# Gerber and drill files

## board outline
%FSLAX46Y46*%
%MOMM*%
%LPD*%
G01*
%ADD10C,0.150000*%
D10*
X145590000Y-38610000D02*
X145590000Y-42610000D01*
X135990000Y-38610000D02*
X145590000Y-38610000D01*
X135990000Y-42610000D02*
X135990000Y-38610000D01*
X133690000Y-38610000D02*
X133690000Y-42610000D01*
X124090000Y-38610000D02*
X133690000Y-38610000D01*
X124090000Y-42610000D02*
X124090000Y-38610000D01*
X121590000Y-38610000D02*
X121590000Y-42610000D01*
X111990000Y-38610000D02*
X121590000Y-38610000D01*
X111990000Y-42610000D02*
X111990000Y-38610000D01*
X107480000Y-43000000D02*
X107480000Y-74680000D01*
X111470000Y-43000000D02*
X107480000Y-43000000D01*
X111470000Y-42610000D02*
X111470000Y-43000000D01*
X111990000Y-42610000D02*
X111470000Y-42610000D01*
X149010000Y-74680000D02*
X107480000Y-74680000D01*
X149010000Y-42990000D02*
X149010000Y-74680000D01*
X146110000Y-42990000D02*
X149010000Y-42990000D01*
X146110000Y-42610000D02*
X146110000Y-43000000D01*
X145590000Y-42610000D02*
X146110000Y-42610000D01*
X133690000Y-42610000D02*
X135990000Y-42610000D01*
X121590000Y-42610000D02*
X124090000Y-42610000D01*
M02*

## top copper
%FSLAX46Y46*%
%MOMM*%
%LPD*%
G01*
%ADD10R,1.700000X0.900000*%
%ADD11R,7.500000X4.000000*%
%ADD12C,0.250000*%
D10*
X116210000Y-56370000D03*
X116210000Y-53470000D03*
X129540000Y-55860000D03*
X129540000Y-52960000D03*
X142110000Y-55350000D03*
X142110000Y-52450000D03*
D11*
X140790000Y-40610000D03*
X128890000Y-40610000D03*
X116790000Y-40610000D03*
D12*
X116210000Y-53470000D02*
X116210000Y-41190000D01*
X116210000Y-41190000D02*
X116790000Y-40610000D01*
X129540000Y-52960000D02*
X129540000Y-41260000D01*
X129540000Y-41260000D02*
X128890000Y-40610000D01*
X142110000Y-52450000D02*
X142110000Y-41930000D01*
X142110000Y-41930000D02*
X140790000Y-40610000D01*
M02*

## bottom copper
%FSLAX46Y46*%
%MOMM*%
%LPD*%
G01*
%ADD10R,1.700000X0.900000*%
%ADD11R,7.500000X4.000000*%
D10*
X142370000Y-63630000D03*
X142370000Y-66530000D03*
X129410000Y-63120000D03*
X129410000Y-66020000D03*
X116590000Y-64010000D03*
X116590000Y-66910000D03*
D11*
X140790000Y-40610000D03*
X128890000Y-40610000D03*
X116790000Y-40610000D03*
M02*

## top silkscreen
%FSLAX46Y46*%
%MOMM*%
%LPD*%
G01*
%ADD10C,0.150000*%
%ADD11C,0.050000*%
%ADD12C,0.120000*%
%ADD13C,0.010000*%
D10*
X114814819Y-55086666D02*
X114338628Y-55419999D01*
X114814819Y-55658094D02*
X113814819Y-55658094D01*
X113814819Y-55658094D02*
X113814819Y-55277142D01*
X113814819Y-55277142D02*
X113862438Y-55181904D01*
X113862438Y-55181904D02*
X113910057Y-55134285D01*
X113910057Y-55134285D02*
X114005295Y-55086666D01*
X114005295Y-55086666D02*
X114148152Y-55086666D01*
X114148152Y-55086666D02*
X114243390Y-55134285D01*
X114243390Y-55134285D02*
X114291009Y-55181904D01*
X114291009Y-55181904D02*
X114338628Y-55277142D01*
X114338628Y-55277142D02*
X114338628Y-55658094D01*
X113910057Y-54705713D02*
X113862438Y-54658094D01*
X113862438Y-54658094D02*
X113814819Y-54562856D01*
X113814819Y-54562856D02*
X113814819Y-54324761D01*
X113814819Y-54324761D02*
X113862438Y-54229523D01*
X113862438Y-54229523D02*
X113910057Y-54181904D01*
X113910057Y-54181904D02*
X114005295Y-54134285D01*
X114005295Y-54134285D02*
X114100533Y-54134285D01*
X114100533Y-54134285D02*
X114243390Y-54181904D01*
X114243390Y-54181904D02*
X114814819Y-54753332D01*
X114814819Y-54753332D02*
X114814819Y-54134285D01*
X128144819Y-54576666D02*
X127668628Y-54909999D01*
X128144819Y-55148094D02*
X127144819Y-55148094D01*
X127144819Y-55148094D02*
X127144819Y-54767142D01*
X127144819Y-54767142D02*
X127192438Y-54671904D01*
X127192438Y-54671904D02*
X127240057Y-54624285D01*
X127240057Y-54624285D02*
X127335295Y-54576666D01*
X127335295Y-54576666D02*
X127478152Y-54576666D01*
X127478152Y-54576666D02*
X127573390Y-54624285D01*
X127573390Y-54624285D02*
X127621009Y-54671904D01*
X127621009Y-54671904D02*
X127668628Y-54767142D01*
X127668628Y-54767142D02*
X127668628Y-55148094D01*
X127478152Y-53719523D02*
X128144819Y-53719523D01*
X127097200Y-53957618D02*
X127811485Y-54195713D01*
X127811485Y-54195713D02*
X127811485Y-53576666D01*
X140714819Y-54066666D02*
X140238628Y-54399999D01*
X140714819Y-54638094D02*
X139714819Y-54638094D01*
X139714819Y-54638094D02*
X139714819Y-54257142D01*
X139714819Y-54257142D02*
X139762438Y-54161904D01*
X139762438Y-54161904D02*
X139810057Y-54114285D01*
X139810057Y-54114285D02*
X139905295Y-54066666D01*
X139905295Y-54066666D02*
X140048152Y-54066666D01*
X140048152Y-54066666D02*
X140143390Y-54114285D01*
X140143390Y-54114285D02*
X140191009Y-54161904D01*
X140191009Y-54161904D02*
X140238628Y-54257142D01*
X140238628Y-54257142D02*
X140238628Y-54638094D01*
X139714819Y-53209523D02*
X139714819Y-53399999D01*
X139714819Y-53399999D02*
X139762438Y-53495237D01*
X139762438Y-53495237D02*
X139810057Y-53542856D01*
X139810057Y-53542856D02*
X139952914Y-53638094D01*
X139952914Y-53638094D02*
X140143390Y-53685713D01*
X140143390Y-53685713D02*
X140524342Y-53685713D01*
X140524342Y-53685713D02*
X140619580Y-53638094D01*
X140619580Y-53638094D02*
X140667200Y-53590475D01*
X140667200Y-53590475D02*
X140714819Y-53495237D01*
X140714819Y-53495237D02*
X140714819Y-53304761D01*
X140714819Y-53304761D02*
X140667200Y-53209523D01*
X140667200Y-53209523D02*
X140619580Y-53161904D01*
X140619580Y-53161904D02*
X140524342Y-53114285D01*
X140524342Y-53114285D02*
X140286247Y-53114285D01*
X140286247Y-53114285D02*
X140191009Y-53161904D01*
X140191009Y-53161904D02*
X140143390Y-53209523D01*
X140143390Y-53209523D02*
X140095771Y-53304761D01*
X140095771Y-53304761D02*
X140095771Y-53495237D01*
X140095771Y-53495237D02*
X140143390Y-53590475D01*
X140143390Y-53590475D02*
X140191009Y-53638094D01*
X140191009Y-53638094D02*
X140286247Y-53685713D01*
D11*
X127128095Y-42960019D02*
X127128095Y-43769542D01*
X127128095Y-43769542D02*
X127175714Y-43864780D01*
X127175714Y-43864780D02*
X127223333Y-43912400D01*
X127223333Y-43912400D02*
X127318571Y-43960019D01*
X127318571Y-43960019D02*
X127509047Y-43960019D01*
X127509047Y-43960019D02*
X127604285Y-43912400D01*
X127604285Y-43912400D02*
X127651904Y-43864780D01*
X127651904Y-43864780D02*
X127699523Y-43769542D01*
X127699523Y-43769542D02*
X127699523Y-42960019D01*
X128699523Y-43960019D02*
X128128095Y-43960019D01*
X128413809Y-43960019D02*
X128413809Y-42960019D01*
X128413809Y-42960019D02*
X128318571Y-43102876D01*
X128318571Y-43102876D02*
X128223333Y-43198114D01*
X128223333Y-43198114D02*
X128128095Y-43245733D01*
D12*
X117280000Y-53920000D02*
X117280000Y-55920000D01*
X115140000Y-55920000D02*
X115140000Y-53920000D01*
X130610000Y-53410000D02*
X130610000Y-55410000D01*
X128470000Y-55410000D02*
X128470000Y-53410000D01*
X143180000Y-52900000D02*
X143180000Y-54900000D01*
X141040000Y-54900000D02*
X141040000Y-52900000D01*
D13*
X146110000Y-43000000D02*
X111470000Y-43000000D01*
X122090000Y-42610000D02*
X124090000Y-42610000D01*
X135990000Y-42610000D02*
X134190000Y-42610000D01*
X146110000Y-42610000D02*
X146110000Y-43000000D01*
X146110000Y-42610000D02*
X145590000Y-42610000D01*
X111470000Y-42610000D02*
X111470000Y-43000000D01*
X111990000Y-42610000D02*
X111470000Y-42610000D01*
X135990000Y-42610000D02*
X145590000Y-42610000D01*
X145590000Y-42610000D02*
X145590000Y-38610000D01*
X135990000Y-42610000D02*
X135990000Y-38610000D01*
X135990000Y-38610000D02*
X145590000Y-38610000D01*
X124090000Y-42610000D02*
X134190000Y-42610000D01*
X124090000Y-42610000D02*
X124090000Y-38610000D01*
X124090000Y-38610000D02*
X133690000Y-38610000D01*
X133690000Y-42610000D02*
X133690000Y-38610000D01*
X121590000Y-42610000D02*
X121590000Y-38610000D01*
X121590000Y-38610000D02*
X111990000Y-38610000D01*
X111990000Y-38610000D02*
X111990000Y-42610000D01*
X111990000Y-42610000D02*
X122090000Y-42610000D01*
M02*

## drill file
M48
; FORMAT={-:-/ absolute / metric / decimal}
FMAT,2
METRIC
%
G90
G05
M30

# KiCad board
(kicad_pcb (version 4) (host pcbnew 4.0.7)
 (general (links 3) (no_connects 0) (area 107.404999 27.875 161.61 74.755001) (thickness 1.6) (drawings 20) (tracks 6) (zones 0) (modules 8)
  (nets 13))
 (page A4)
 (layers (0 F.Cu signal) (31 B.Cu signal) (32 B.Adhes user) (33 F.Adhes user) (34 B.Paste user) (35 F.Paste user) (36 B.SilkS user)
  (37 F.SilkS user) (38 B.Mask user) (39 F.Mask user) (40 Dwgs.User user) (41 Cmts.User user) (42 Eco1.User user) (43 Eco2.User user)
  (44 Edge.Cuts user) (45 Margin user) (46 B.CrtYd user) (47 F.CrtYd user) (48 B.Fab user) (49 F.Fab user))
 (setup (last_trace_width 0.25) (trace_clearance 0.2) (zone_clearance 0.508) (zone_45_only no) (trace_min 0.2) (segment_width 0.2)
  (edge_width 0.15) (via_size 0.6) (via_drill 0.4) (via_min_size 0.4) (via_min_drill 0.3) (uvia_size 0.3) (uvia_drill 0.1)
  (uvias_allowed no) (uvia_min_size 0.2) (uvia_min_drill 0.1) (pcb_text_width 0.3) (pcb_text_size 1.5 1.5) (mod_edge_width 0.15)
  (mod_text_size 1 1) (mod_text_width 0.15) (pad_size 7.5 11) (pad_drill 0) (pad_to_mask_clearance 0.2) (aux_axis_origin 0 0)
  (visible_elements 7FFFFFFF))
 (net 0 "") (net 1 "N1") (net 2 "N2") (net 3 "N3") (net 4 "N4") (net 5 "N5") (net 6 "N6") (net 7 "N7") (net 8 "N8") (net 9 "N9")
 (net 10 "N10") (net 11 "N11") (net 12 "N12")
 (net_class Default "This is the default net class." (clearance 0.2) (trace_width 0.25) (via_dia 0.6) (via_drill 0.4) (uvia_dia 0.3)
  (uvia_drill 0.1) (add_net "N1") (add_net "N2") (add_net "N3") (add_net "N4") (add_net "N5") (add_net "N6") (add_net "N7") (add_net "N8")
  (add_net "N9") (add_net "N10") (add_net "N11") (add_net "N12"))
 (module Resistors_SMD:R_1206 (layer B.Cu) (at 142.37 65.08 270)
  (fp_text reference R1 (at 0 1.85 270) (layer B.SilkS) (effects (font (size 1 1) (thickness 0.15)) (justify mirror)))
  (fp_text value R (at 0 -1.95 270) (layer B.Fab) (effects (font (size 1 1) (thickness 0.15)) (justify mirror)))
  (pad 1 smd rect (at -1.45 0 270) (size 0.9 1.7) (layers B.Cu B.Paste B.Mask) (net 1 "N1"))
  (pad 2 smd rect (at 1.45 0 270) (size 0.9 1.7) (layers B.Cu B.Paste B.Mask) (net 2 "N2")))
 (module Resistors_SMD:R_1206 (layer F.Cu) (at 116.21 54.92 90)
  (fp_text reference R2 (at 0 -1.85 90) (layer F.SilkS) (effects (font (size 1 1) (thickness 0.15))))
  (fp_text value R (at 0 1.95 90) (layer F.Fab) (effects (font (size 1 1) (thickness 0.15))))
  (fp_line (start 1 1.07) (end -1 1.07) (layer F.SilkS) (width 0.12))
  (fp_line (start -1 -1.07) (end 1 -1.07) (layer F.SilkS) (width 0.12))
  (pad 1 smd rect (at -1.45 0 90) (size 0.9 1.7) (layers F.Cu F.Paste F.Mask) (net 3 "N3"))
  (pad 2 smd rect (at 1.45 0 90) (size 0.9 1.7) (layers F.Cu F.Paste F.Mask) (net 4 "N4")))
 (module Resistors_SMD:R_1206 (layer B.Cu) (at 129.41 64.57 270)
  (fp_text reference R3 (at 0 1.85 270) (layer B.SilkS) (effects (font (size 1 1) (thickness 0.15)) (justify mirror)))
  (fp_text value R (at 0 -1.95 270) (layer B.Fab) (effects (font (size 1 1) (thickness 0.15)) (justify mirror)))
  (pad 1 smd rect (at -1.45 0 270) (size 0.9 1.7) (layers B.Cu B.Paste B.Mask) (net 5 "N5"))
  (pad 2 smd rect (at 1.45 0 270) (size 0.9 1.7) (layers B.Cu B.Paste B.Mask) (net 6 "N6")))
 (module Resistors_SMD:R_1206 (layer F.Cu) (at 129.54 54.41 90)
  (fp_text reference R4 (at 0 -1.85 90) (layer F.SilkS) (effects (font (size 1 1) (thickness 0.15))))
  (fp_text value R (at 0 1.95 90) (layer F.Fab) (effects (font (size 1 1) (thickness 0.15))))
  (fp_line (start 1 1.07) (end -1 1.07) (layer F.SilkS) (width 0.12))
  (fp_line (start -1 -1.07) (end 1 -1.07) (layer F.SilkS) (width 0.12))
  (pad 1 smd rect (at -1.45 0 90) (size 0.9 1.7) (layers F.Cu F.Paste F.Mask) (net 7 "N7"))
  (pad 2 smd rect (at 1.45 0 90) (size 0.9 1.7) (layers F.Cu F.Paste F.Mask) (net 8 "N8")))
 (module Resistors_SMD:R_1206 (layer B.Cu) (at 116.59 65.46 270)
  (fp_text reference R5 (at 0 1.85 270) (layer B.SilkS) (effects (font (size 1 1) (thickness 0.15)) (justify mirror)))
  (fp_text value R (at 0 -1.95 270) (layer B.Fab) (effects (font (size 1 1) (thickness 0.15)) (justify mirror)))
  (pad 1 smd rect (at -1.45 0 270) (size 0.9 1.7) (layers B.Cu B.Paste B.Mask) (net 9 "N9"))
  (pad 2 smd rect (at 1.45 0 270) (size 0.9 1.7) (layers B.Cu B.Paste B.Mask) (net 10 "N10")))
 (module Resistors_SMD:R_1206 (layer F.Cu) (at 142.11 53.9 90)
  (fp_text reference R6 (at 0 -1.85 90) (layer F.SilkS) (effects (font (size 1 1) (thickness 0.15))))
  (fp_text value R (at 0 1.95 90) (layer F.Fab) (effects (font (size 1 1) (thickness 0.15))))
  (fp_line (start 1 1.07) (end -1 1.07) (layer F.SilkS) (width 0.12))
  (fp_line (start -1 -1.07) (end 1 -1.07) (layer F.SilkS) (width 0.12))
  (pad 1 smd rect (at -1.45 0 90) (size 0.9 1.7) (layers F.Cu F.Paste F.Mask) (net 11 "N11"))
  (pad 2 smd rect (at 1.45 0 90) (size 0.9 1.7) (layers F.Cu F.Paste F.Mask) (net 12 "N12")))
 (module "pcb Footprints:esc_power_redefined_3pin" (layer F.Cu) (at 111.99 42.61)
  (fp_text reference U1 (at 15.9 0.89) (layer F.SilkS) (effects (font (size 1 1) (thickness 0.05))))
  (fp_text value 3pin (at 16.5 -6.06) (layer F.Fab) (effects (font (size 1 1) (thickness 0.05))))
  (fp_line (start 34.12 0.39) (end -0.52 0.39) (layer F.SilkS) (width 0.01))
  (fp_line (start 10.1 0) (end 12.1 0) (layer F.SilkS) (width 0.01))
  (fp_line (start 24 0) (end 22.2 0) (layer F.SilkS) (width 0.01))
  (fp_line (start 34.12 0) (end 34.12 0.39) (layer F.SilkS) (width 0.01))
  (fp_line (start 34.12 0) (end 33.6 0) (layer F.SilkS) (width 0.01))
  (fp_line (start -0.52 0) (end -0.52 0.39) (layer F.SilkS) (width 0.01))
  (fp_line (start 0 0) (end -0.52 0) (layer F.SilkS) (width 0.01))
  (fp_line (start 24 0) (end 33.6 0) (layer F.SilkS) (width 0.01))
  (fp_line (start 33.6 0) (end 33.6 -4) (layer F.SilkS) (width 0.01))
  (fp_line (start 24 0) (end 24 -4) (layer F.SilkS) (width 0.01))
  (fp_line (start 24 -4) (end 33.6 -4) (layer F.SilkS) (width 0.01))
  (fp_line (start 12.1 0) (end 22.2 0) (layer F.SilkS) (width 0.01))
  (fp_line (start 12.1 0) (end 12.1 -4) (layer F.SilkS) (width 0.01))
  (fp_line (start 12.1 -4) (end 21.7 -4) (layer F.SilkS) (width 0.01))
  (fp_line (start 21.7 0) (end 21.7 -4) (layer F.SilkS) (width 0.01))
  (fp_line (start 9.6 0) (end 9.6 -4) (layer F.SilkS) (width 0.01))
  (fp_line (start 9.6 -4) (end 0 -4) (layer F.SilkS) (width 0.01))
  (fp_line (start 0 -4) (end 0 0) (layer F.SilkS) (width 0.01))
  (fp_line (start 0 0) (end 10.1 0) (layer F.SilkS) (width 0.01))
  (pad 3 smd rect (at 28.8 -2) (size 7.5 4) (layers F.Cu B.Adhes F.Mask) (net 12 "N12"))
  (pad 2 smd rect (at 16.9 -2) (size 7.5 4) (layers F.Cu B.Adhes F.Mask) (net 8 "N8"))
  (pad 1 smd rect (at 4.8 -2) (size 7.5 4) (layers F.Cu B.Adhes F.Mask) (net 4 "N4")))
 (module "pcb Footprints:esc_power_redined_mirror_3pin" (layer B.Cu) (at 152.8 42.61 180)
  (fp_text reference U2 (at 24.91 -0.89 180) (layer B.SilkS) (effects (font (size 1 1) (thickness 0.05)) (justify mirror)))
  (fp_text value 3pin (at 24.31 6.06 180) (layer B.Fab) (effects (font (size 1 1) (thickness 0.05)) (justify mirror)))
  (pad 3 smd rect (at 12.01 2 180) (size 7.5 4) (layers B.Cu F.Adhes B.Mask))
  (pad 2 smd rect (at 23.91 2 180) (size 7.5 4) (layers B.Cu F.Adhes B.Mask))
  (pad 1 smd rect (at 36.01 2 180) (size 7.5 4) (layers B.Cu F.Adhes B.Mask)))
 (gr_line (start 145.59 38.61) (end 145.59 42.61) (angle 90) (layer Edge.Cuts) (width 0.15))
 (gr_line (start 135.99 38.61) (end 145.59 38.61) (angle 90) (layer Edge.Cuts) (width 0.15))
 (gr_line (start 135.99 42.61) (end 135.99 38.61) (angle 90) (layer Edge.Cuts) (width 0.15))
 (gr_line (start 133.69 38.61) (end 133.69 42.61) (angle 90) (layer Edge.Cuts) (width 0.15))
 (gr_line (start 124.09 38.61) (end 133.69 38.61) (angle 90) (layer Edge.Cuts) (width 0.15))
 (gr_line (start 124.09 42.61) (end 124.09 38.61) (angle 90) (layer Edge.Cuts) (width 0.15))
 (gr_line (start 121.59 38.61) (end 121.59 42.61) (angle 90) (layer Edge.Cuts) (width 0.15))
 (gr_line (start 111.99 38.61) (end 121.59 38.61) (angle 90) (layer Edge.Cuts) (width 0.15))
 (gr_line (start 111.99 42.61) (end 111.99 38.61) (angle 90) (layer Edge.Cuts) (width 0.15))
 (gr_line (start 107.48 43) (end 107.48 74.68) (angle 90) (layer Edge.Cuts) (width 0.15))
 (gr_line (start 111.47 43) (end 107.48 43) (angle 90) (layer Edge.Cuts) (width 0.15))
 (gr_line (start 111.47 42.61) (end 111.47 43) (angle 90) (layer Edge.Cuts) (width 0.15))
 (gr_line (start 111.99 42.61) (end 111.47 42.61) (angle 90) (layer Edge.Cuts) (width 0.15))
 (gr_line (start 149.01 74.68) (end 107.48 74.68) (angle 90) (layer Edge.Cuts) (width 0.15))
 (gr_line (start 149.01 42.99) (end 149.01 74.68) (angle 90) (layer Edge.Cuts) (width 0.15))
 (gr_line (start 146.11 42.99) (end 149.01 42.99) (angle 90) (layer Edge.Cuts) (width 0.15))
 (gr_line (start 146.11 42.61) (end 146.11 43) (angle 90) (layer Edge.Cuts) (width 0.15))
 (gr_line (start 145.59 42.61) (end 146.11 42.61) (angle 90) (layer Edge.Cuts) (width 0.15))
 (gr_line (start 133.69 42.61) (end 135.99 42.61) (angle 90) (layer Edge.Cuts) (width 0.15))
 (gr_line (start 121.59 42.61) (end 124.09 42.61) (angle 90) (layer Edge.Cuts) (width 0.15))
 (segment (start 116.21 53.47) (end 116.21 41.19) (width 0.25) (layer F.Cu) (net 4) (status C00000))
 (segment (start 116.21 41.19) (end 116.79 40.61) (width 0.25) (layer F.Cu) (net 4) (status C00000))
 (segment (start 129.54 52.96) (end 129.54 41.26) (width 0.25) (layer F.Cu) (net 8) (status C00000))
 (segment (start 129.54 41.26) (end 128.89 40.61) (width 0.25) (layer F.Cu) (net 8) (status C00000))
 (segment (start 142.11 52.45) (end 142.11 41.93) (width 0.25) (layer F.Cu) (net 12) (status C00000))
 (segment (start 142.11 41.93) (end 140.79 40.61) (width 0.25) (layer F.Cu) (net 12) (status C00000)))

